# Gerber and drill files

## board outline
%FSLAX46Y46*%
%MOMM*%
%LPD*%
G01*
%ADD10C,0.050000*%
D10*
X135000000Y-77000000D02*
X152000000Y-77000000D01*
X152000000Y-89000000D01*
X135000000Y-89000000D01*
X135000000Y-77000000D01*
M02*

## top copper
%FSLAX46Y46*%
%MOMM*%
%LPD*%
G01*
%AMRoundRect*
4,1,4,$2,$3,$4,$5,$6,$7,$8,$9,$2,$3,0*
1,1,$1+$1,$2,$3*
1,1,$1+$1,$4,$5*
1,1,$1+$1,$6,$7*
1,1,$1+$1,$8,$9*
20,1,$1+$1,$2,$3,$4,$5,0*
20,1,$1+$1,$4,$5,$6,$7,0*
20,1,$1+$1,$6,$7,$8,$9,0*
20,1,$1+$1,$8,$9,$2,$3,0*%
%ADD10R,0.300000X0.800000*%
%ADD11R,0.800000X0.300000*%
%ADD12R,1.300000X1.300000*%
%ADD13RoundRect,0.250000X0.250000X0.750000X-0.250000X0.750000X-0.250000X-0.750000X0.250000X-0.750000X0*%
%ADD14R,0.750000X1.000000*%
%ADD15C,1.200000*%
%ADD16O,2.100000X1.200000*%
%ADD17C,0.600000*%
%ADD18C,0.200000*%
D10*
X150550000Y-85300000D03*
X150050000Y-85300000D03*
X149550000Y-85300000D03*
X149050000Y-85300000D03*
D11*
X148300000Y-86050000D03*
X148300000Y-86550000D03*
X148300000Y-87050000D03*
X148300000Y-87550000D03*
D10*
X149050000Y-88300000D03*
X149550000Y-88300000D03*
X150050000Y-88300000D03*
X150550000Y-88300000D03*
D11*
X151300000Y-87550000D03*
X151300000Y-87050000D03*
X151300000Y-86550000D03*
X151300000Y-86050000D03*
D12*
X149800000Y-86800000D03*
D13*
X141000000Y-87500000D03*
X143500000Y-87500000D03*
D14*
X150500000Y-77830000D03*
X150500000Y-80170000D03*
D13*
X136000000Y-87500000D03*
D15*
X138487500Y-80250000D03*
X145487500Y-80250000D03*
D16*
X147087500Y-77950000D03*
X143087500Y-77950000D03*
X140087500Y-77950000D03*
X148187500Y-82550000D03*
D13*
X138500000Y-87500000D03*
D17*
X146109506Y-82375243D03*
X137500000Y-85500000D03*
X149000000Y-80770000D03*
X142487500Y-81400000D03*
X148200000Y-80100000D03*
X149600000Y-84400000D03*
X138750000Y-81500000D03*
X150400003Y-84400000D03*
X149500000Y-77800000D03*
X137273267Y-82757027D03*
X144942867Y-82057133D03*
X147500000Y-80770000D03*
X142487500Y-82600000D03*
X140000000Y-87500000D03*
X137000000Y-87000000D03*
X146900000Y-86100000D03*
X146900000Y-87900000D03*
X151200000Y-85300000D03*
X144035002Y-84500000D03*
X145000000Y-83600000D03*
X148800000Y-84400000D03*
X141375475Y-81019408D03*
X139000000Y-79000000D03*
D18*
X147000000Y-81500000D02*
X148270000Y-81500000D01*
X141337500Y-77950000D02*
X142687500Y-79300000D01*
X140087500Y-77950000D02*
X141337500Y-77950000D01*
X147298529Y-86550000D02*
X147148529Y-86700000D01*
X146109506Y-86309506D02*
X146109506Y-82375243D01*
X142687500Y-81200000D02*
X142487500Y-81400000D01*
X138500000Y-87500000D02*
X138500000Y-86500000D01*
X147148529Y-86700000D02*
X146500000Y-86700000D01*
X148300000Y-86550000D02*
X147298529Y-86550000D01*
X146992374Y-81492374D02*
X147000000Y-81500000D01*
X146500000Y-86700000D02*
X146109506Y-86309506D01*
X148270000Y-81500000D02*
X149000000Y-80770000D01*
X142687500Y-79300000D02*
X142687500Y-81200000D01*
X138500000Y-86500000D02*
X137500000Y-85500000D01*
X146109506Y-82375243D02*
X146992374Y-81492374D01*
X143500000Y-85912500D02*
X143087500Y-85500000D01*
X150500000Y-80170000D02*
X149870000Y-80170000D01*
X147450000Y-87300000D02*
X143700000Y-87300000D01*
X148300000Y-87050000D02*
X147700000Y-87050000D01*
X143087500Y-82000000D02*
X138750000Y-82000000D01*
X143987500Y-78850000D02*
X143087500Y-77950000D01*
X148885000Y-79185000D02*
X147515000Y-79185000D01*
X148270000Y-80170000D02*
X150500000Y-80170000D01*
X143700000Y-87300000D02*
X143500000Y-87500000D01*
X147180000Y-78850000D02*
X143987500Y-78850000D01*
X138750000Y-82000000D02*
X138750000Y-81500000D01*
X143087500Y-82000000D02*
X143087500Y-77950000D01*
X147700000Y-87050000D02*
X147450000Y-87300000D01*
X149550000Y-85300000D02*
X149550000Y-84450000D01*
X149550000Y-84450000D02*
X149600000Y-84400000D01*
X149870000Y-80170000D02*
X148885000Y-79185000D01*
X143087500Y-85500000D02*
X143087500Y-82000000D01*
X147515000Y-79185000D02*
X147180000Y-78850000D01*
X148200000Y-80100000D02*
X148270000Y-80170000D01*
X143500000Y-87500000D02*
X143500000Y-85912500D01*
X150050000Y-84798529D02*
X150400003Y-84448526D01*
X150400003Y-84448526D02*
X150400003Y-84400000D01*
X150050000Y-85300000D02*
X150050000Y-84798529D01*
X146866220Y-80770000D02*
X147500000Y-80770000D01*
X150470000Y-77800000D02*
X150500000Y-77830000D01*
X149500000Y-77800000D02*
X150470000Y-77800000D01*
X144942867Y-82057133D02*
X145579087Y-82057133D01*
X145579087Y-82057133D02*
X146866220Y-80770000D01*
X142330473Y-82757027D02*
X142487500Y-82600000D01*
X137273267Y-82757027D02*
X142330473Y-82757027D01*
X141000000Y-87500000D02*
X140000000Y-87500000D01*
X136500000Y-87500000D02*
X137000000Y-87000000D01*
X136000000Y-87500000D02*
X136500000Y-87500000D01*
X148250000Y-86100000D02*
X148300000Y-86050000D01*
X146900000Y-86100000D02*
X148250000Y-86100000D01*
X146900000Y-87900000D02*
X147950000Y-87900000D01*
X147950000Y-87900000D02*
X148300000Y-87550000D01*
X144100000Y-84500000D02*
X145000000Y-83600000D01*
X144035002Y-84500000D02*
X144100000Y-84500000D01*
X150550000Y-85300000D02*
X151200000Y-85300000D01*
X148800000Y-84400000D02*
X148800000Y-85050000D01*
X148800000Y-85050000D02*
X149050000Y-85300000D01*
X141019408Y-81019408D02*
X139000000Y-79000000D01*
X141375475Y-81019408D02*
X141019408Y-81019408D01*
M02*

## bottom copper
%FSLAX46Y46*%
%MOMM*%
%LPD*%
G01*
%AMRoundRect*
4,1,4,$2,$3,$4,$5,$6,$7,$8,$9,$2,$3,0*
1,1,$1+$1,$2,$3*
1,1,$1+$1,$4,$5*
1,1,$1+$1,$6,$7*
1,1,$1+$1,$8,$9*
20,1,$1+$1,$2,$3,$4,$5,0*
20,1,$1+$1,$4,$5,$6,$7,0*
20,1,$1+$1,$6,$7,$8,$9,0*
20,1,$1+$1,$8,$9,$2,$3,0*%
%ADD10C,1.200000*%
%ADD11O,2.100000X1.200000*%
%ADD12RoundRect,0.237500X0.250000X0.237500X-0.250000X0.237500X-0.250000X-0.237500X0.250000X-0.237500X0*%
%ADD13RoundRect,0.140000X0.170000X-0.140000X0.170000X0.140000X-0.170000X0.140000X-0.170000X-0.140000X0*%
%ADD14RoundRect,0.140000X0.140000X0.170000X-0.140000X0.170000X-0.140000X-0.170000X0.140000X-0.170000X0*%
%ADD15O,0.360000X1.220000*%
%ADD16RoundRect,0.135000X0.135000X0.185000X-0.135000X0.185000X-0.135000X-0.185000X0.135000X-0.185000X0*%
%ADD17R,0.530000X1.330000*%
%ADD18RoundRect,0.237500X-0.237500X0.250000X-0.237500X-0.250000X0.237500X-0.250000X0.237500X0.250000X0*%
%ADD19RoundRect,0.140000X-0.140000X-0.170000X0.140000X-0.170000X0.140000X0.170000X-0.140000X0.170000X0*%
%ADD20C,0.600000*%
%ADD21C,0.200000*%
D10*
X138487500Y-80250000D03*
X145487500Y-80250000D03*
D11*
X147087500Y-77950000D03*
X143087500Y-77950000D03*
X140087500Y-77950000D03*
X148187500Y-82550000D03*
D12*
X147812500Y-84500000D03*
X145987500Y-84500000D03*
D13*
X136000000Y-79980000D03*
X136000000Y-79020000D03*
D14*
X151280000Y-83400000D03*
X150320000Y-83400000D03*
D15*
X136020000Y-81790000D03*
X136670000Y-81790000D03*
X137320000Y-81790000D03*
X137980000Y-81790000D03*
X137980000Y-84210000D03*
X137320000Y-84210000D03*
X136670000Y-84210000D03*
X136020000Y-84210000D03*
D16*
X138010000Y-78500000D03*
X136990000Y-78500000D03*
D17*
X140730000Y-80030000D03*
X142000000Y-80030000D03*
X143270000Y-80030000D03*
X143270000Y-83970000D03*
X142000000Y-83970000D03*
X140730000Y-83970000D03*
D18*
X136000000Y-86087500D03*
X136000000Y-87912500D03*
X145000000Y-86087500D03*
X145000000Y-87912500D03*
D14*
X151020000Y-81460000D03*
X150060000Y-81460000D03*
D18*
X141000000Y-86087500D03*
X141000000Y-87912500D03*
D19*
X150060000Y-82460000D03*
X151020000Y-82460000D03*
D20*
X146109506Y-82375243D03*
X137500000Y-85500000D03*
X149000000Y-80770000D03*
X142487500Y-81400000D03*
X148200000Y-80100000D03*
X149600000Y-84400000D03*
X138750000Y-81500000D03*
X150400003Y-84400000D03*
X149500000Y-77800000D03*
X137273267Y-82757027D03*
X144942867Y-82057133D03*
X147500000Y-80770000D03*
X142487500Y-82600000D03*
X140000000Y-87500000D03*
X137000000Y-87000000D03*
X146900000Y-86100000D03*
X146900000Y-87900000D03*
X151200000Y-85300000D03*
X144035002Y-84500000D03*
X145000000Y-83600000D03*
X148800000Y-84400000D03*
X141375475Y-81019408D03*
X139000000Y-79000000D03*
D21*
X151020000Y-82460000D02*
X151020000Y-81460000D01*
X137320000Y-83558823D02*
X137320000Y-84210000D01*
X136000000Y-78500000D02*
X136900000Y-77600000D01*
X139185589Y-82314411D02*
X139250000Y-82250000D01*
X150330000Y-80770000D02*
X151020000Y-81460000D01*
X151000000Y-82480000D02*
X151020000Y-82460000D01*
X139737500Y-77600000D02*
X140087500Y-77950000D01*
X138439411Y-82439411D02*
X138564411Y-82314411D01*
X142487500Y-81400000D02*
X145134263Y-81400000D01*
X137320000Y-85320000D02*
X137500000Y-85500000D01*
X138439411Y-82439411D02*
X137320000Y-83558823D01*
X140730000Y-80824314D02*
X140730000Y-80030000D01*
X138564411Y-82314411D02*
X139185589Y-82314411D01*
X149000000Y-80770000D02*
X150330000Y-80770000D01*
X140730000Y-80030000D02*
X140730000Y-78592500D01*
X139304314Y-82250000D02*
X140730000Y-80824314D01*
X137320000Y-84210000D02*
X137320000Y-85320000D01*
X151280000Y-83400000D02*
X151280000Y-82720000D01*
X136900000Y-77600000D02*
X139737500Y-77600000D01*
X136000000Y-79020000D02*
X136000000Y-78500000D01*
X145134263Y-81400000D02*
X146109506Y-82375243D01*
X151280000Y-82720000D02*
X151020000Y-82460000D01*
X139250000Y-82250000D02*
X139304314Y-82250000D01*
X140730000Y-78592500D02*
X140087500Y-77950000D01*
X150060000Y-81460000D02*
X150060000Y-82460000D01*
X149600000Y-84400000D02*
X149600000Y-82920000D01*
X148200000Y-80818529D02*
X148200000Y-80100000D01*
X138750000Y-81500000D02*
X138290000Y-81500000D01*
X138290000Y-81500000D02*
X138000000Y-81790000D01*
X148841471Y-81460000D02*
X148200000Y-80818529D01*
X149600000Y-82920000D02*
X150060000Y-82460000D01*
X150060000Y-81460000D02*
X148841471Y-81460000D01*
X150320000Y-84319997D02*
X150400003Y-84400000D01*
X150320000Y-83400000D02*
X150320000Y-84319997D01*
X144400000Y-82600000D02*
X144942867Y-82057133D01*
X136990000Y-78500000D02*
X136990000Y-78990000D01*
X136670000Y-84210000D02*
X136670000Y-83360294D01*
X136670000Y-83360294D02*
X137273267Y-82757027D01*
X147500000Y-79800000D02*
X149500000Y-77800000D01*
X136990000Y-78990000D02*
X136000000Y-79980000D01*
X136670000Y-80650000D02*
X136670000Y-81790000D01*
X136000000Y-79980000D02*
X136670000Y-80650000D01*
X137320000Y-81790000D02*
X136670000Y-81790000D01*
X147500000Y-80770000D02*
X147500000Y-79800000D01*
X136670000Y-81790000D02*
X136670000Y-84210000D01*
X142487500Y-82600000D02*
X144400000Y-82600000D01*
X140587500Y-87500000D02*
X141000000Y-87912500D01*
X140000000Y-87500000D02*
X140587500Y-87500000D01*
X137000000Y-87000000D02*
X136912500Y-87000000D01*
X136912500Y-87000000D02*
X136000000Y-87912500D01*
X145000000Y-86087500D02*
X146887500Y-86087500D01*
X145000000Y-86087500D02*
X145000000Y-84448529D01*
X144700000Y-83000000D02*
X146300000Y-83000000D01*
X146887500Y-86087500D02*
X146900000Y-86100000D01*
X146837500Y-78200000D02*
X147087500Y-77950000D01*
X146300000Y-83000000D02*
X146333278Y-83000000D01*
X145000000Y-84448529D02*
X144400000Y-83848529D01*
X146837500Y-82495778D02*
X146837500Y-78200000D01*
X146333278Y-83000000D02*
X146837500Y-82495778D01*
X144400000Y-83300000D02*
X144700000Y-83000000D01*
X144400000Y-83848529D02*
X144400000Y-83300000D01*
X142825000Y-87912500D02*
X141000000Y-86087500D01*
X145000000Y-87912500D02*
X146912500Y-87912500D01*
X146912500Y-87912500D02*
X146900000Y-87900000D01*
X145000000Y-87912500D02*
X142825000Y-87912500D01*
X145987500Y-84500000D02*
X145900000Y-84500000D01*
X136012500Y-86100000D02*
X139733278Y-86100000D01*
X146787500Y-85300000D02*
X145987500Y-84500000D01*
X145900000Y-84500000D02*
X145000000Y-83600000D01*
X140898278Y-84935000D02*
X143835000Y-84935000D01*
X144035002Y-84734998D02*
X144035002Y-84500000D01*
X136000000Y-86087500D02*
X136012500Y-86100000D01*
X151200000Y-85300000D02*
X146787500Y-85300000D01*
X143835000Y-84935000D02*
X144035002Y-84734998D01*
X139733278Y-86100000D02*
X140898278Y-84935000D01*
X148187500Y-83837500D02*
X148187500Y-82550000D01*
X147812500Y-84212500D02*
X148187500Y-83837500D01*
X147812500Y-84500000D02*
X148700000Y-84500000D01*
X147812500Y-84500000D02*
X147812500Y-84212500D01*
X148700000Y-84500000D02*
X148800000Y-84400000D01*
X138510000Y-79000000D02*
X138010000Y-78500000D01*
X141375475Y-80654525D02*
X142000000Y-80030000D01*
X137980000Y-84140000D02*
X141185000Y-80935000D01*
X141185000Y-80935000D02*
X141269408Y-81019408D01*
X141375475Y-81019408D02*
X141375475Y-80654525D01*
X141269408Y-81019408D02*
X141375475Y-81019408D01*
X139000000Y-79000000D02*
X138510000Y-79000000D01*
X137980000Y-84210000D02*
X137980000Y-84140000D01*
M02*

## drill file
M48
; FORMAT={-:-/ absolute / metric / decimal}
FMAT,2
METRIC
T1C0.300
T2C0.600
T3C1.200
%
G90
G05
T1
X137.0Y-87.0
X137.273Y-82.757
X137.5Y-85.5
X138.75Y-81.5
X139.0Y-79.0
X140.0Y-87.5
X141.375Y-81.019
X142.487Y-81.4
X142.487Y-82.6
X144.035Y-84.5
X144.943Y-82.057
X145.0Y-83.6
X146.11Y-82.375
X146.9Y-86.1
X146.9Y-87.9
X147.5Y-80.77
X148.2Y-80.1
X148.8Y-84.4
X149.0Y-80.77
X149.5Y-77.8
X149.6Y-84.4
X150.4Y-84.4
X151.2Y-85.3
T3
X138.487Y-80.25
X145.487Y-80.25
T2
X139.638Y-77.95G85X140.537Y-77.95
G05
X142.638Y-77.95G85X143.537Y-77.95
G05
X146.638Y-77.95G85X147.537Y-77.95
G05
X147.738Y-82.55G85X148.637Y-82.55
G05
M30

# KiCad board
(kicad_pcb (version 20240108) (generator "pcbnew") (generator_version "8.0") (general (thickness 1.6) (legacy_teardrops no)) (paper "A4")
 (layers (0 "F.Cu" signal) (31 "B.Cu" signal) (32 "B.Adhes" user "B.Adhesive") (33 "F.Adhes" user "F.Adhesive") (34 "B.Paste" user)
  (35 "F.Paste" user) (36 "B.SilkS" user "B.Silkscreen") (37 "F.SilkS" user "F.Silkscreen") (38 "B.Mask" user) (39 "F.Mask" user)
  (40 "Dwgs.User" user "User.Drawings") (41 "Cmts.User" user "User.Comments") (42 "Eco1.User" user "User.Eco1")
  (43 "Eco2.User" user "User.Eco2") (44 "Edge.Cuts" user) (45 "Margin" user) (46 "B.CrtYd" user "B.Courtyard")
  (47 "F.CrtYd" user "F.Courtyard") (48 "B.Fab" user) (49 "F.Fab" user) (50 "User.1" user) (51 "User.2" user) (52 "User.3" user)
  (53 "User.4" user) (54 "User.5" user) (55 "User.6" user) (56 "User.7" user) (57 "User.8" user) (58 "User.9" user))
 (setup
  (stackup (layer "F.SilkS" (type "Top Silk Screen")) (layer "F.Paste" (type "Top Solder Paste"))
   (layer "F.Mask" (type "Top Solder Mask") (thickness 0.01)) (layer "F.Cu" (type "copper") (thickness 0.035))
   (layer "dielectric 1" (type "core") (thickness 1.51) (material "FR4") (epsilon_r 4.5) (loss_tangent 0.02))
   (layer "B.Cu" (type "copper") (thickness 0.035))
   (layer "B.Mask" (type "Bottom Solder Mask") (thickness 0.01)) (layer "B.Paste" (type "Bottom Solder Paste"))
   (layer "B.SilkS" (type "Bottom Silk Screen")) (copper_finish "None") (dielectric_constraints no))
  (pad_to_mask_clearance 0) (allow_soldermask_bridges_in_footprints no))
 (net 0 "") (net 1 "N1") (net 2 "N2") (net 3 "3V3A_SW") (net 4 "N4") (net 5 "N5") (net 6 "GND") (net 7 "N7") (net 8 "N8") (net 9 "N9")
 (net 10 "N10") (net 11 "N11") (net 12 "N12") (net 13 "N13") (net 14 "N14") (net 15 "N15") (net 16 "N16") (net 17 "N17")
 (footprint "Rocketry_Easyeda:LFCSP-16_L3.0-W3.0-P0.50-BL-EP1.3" (layer "F.Cu") (at 149.8 86.8 180)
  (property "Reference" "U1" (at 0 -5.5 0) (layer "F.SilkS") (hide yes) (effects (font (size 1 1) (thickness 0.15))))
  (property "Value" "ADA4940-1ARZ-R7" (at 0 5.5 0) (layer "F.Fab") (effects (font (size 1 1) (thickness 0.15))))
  (pad "1" smd rect (at -0.75 1.5) (size 0.3 0.8) (layers "F.Cu" "F.Paste" "F.Mask") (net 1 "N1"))
  (pad "2" smd rect (at -0.25 1.5) (size 0.3 0.8) (layers "F.Cu" "F.Paste" "F.Mask") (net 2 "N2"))
  (pad "3" smd rect (at 0.25 1.5) (size 0.3 0.8) (layers "F.Cu" "F.Paste" "F.Mask") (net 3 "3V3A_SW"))
  (pad "4" smd rect (at 0.75 1.5) (size 0.3 0.8) (layers "F.Cu" "F.Paste" "F.Mask") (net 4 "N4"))
  (pad "5" smd rect (at 1.5 0.75 270) (size 0.3 0.8) (layers "F.Cu" "F.Paste" "F.Mask") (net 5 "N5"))
  (pad "6" smd rect (at 1.5 0.25 270) (size 0.3 0.8) (layers "F.Cu" "F.Paste" "F.Mask") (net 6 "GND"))
  (pad "7" smd rect (at 1.5 -0.25 270) (size 0.3 0.8) (layers "F.Cu" "F.Paste" "F.Mask") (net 3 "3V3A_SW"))
  (pad "8" smd rect (at 1.5 -0.75 270) (size 0.3 0.8) (layers "F.Cu" "F.Paste" "F.Mask") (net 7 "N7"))
  (pad "9" smd rect (at 0.75 -1.5) (size 0.3 0.8) (layers "F.Cu" "F.Paste" "F.Mask"))
  (pad "10" smd rect (at 0.25 -1.5) (size 0.3 0.8) (layers "F.Cu" "F.Paste" "F.Mask"))
  (pad "11" smd rect (at -0.25 -1.5) (size 0.3 0.8) (layers "F.Cu" "F.Paste" "F.Mask"))
  (pad "12" smd rect (at -0.75 -1.5) (size 0.3 0.8) (layers "F.Cu" "F.Paste" "F.Mask"))
  (pad "13" smd rect (at -1.5 -0.75 270) (size 0.3 0.8) (layers "F.Cu" "F.Paste" "F.Mask"))
  (pad "14" smd rect (at -1.5 -0.25 270) (size 0.3 0.8) (layers "F.Cu" "F.Paste" "F.Mask"))
  (pad "15" smd rect (at -1.5 0.25 270) (size 0.3 0.8) (layers "F.Cu" "F.Paste" "F.Mask"))
  (pad "16" smd rect (at -1.5 0.75 270) (size 0.3 0.8) (layers "F.Cu" "F.Paste" "F.Mask"))
  (pad "17" smd rect (at 0 0) (size 1.3 1.3) (layers "F.Cu" "F.Paste" "F.Mask")))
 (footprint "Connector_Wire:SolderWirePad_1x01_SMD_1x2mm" (layer "F.Cu") (at 141 87.5 180)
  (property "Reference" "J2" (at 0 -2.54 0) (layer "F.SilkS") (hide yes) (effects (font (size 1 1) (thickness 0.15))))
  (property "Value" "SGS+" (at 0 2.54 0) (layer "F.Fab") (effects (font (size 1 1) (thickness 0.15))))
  (pad "1" smd roundrect (at 0 0 180) (size 1 2) (layers "F.Cu" "F.Paste" "F.Mask") (roundrect_rratio 0.25) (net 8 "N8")))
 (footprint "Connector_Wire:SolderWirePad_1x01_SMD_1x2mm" (layer "F.Cu") (at 143.5 87.5 180)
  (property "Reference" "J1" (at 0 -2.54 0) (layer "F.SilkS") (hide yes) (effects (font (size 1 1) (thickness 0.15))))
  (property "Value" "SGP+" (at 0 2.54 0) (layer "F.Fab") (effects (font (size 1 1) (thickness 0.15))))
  (pad "1" smd roundrect (at 0 0 180) (size 1 2) (layers "F.Cu" "F.Paste" "F.Mask") (roundrect_rratio 0.25) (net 3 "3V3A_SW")))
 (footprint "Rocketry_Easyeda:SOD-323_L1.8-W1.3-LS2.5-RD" (layer "F.Cu") (at 150.5 79 -90)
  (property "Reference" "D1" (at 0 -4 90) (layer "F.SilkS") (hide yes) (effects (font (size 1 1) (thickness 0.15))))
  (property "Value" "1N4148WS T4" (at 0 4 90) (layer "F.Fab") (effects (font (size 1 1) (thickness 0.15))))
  (pad "1" smd rect (at -1.17 0 270) (size 1 0.75) (layers "F.Cu" "F.Paste" "F.Mask") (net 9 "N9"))
  (pad "2" smd rect (at 1.17 0 270) (size 1 0.75) (layers "F.Cu" "F.Paste" "F.Mask") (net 3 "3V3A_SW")))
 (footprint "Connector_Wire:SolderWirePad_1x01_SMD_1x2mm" (layer "F.Cu") (at 136 87.5 180)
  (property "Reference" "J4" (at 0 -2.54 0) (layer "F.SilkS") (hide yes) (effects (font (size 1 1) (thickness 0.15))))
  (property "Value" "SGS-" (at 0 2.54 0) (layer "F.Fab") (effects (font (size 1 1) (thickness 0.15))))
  (pad "1" smd roundrect (at 0 0 180) (size 1 2) (layers "F.Cu" "F.Paste" "F.Mask") (roundrect_rratio 0.25) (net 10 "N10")))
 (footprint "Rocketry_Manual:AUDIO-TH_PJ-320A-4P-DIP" (layer "F.Cu") (at 144.1375 80.25)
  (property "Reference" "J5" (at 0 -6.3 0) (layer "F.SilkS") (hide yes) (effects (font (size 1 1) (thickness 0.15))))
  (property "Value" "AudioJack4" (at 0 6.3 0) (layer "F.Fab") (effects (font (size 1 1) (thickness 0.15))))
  (pad "" thru_hole circle (at -5.65 0) (size 1.2 1.2) (drill 1.2) (layers "*.Cu" "*.Mask") (remove_unused_layers no))
  (pad "" thru_hole circle (at 1.35 0) (size 1.2 1.2) (drill 1.2) (layers "*.Cu" "*.Mask") (remove_unused_layers no))
  (pad "R1" thru_hole oval (at 2.95 -2.3 90) (size 1.2 2.1) (drill oval 0.599999 1.499997) (layers "*.Cu" "*.Mask")
   (remove_unused_layers no) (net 5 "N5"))
  (pad "R2" thru_hole oval (at -1.05 -2.3 90) (size 1.2 2.1) (drill oval 0.599999 1.499997) (layers "*.Cu" "*.Mask")
   (remove_unused_layers no) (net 3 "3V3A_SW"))
  (pad "S" thru_hole oval (at -4.05 -2.3 90) (size 1.2 2.1) (drill oval 0.599999 1.499997) (layers "*.Cu" "*.Mask")
   (remove_unused_layers no) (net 6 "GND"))
  (pad "T" thru_hole oval (at 4.05 2.3 90) (size 1.2 2.1) (drill oval 0.599999 1.499997) (layers "*.Cu" "*.Mask") (remove_unused_layers no)
   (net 4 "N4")))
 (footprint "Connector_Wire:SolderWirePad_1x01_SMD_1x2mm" (layer "F.Cu") (at 138.5 87.5 180)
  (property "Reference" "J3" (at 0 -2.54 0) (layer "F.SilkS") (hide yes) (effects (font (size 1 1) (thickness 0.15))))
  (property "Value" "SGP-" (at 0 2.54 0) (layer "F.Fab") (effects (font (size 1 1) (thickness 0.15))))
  (pad "1" smd roundrect (at 0 0 180) (size 1 2) (layers "F.Cu" "F.Paste" "F.Mask") (roundrect_rratio 0.25) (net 6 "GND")))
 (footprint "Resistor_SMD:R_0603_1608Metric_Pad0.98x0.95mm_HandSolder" (layer "B.Cu") (at 146.9 84.5 180)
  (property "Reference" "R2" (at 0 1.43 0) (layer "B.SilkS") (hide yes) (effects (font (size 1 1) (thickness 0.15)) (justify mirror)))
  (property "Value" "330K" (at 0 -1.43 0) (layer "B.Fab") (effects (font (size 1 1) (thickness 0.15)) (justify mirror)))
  (pad "1" smd roundrect (at -0.9125 0 180) (size 0.975 0.95) (layers "B.Cu" "B.Paste" "B.Mask") (roundrect_rratio 0.25) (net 4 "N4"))
  (pad "2" smd roundrect (at 0.9125 0 180) (size 0.975 0.95) (layers "B.Cu" "B.Paste" "B.Mask") (roundrect_rratio 0.25) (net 1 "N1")))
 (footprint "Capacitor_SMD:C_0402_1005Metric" (layer "B.Cu") (at 136 79.5 90)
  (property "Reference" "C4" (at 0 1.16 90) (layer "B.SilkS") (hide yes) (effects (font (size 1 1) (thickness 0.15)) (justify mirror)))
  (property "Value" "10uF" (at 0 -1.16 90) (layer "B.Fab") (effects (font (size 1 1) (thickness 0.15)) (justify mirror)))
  (pad "1" smd roundrect (at -0.48 0 90) (size 0.56 0.62) (layers "B.Cu" "B.Paste" "B.Mask") (roundrect_rratio 0.25) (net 9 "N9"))
  (pad "2" smd roundrect (at 0.48 0 90) (size 0.56 0.62) (layers "B.Cu" "B.Paste" "B.Mask") (roundrect_rratio 0.25) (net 6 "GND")))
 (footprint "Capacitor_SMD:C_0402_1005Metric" (layer "B.Cu") (at 150.8 83.4 180)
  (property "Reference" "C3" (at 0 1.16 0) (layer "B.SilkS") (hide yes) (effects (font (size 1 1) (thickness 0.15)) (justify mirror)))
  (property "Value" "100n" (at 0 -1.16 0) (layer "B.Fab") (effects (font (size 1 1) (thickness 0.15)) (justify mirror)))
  (pad "1" smd roundrect (at -0.48 0 180) (size 0.56 0.62) (layers "B.Cu" "B.Paste" "B.Mask") (roundrect_rratio 0.25) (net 6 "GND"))
  (pad "2" smd roundrect (at 0.48 0 180) (size 0.56 0.62) (layers "B.Cu" "B.Paste" "B.Mask") (roundrect_rratio 0.25) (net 2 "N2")))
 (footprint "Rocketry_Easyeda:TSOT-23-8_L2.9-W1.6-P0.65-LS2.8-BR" (layer "B.Cu") (at 137 83 90)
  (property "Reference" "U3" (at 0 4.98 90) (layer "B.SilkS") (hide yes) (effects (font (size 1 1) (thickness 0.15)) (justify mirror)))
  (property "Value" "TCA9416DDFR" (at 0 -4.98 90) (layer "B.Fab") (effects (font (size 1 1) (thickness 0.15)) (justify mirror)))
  (pad "1" smd oval (at 1.21 -0.98 90) (size 1.22 0.36) (layers "B.Cu" "B.Paste" "B.Mask") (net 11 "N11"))
  (pad "2" smd oval (at 1.21 -0.33 90) (size 1.22 0.36) (layers "B.Cu" "B.Paste" "B.Mask") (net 9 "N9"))
  (pad "3" smd oval (at 1.21 0.32 90) (size 1.22 0.36) (layers "B.Cu" "B.Paste" "B.Mask") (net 9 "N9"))
  (pad "4" smd oval (at 1.21 0.98 90) (size 1.22 0.36) (layers "B.Cu" "B.Paste" "B.Mask") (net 3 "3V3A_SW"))
  (pad "5" smd oval (at -1.21 0.98 90) (size 1.22 0.36) (layers "B.Cu" "B.Paste" "B.Mask") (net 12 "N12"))
  (pad "6" smd oval (at -1.21 0.32 90) (size 1.22 0.36) (layers "B.Cu" "B.Paste" "B.Mask") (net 6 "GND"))
  (pad "7" smd oval (at -1.21 -0.33 90) (size 1.22 0.36) (layers "B.Cu" "B.Paste" "B.Mask") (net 9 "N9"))
  (pad "8" smd oval (at -1.21 -0.98 90) (size 1.22 0.36) (layers "B.Cu" "B.Paste" "B.Mask") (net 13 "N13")))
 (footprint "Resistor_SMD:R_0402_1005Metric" (layer "B.Cu") (at 137.5 78.5 180)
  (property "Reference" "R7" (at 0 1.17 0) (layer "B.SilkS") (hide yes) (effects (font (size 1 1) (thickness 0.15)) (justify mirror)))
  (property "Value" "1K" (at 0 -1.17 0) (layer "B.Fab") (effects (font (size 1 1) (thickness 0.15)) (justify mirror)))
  (pad "1" smd roundrect (at -0.51 0 180) (size 0.54 0.64) (layers "B.Cu" "B.Paste" "B.Mask") (roundrect_rratio 0.25) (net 12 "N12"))
  (pad "2" smd roundrect (at 0.51 0 180) (size 0.54 0.64) (layers "B.Cu" "B.Paste" "B.Mask") (roundrect_rratio 0.25) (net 9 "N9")))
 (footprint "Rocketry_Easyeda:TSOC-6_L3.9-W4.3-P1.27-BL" (layer "B.Cu") (at 142 82)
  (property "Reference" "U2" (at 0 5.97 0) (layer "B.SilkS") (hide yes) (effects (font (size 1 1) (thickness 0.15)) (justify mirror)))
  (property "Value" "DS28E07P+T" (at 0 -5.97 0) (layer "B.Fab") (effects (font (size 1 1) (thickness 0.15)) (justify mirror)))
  (pad "1" smd rect (at -1.27 -1.97) (size 0.53 1.33) (layers "B.Cu" "B.Paste" "B.Mask") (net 6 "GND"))
  (pad "2" smd rect (at 0 -1.97) (size 0.53 1.33) (layers "B.Cu" "B.Paste" "B.Mask") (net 12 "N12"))
  (pad "3" smd rect (at 1.27 -1.97) (size 0.53 1.33) (layers "B.Cu" "B.Paste" "B.Mask") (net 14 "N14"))
  (pad "4" smd rect (at 1.27 1.97) (size 0.53 1.33) (layers "B.Cu" "B.Paste" "B.Mask") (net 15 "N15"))
  (pad "5" smd rect (at 0 1.97) (size 0.53 1.33) (layers "B.Cu" "B.Paste" "B.Mask") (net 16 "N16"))
  (pad "6" smd rect (at -1.27 1.97) (size 0.53 1.33) (layers "B.Cu" "B.Paste" "B.Mask") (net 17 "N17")))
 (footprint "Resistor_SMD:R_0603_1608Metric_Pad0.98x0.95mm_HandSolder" (layer "B.Cu") (at 136 87 -90)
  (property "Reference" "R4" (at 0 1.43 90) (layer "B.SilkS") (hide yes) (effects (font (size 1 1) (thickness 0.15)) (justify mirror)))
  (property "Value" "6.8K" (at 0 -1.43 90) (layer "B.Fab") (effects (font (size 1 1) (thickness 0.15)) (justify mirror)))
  (pad "1" smd roundrect (at -0.9125 0 270) (size 0.975 0.95) (layers "B.Cu" "B.Paste" "B.Mask") (roundrect_rratio 0.25) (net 1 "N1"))
  (pad "2" smd roundrect (at 0.9125 0 270) (size 0.975 0.95) (layers "B.Cu" "B.Paste" "B.Mask") (roundrect_rratio 0.25) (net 10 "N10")))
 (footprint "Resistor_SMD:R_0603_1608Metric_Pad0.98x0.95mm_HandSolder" (layer "B.Cu") (at 145 87 -90)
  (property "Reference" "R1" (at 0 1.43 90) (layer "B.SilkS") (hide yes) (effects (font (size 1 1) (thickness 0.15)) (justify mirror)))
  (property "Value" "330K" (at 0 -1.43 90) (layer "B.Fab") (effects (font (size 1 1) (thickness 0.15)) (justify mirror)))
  (pad "1" smd roundrect (at -0.9125 0 270) (size 0.975 0.95) (layers "B.Cu" "B.Paste" "B.Mask") (roundrect_rratio 0.25) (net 5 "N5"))
  (pad "2" smd roundrect (at 0.9125 0 270) (size 0.975 0.95) (layers "B.Cu" "B.Paste" "B.Mask") (roundrect_rratio 0.25) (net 7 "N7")))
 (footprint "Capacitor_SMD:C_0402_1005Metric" (layer "B.Cu") (at 150.54 81.46 180)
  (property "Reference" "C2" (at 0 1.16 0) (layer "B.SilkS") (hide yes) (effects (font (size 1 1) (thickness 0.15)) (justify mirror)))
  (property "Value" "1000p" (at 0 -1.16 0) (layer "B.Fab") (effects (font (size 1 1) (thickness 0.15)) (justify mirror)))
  (pad "1" smd roundrect (at -0.48 0 180) (size 0.56 0.62) (layers "B.Cu" "B.Paste" "B.Mask") (roundrect_rratio 0.25) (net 6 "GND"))
  (pad "2" smd roundrect (at 0.48 0 180) (size 0.56 0.62) (layers "B.Cu" "B.Paste" "B.Mask") (roundrect_rratio 0.25) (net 3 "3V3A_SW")))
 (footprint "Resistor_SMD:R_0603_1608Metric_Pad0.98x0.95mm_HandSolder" (layer "B.Cu") (at 141 87 -90)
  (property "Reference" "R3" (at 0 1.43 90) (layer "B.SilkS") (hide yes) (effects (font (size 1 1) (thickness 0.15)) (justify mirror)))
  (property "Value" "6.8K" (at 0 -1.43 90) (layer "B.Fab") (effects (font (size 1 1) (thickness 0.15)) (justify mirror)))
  (pad "1" smd roundrect (at -0.9125 0 270) (size 0.975 0.95) (layers "B.Cu" "B.Paste" "B.Mask") (roundrect_rratio 0.25) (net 7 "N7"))
  (pad "2" smd roundrect (at 0.9125 0 270) (size 0.975 0.95) (layers "B.Cu" "B.Paste" "B.Mask") (roundrect_rratio 0.25) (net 8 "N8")))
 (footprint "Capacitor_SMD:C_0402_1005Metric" (layer "B.Cu") (at 150.54 82.46)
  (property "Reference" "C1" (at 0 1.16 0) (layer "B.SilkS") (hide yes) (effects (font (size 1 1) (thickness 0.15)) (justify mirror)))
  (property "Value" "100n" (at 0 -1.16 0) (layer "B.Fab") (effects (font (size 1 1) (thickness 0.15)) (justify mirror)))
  (pad "1" smd roundrect (at -0.48 0) (size 0.56 0.62) (layers "B.Cu" "B.Paste" "B.Mask") (roundrect_rratio 0.25) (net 3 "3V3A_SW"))
  (pad "2" smd roundrect (at 0.48 0) (size 0.56 0.62) (layers "B.Cu" "B.Paste" "B.Mask") (roundrect_rratio 0.25) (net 6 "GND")))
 (gr_rect (start 135 77) (end 152 89) (stroke (width 0.05) (type default)) (fill none) (layer "Edge.Cuts"))
 (segment (start 147 81.5) (end 148.27 81.5) (width 0.2) (layer "F.Cu") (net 6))
 (segment (start 141.3375 77.95) (end 142.6875 79.3) (width 0.2) (layer "F.Cu") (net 6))
 (segment (start 140.0875 77.95) (end 141.3375 77.95) (width 0.2) (layer "F.Cu") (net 6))
 (segment (start 147.298529 86.55) (end 147.148529 86.7) (width 0.2) (layer "F.Cu") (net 6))
 (segment (start 146.109506 86.309506) (end 146.109506 82.375243) (width 0.2) (layer "F.Cu") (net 6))
 (segment (start 142.6875 81.2) (end 142.4875 81.4) (width 0.2) (layer "F.Cu") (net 6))
 (segment (start 138.5 87.5) (end 138.5 86.5) (width 0.2) (layer "F.Cu") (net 6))
 (segment (start 147.148529 86.7) (end 146.5 86.7) (width 0.2) (layer "F.Cu") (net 6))
 (segment (start 148.3 86.55) (end 147.298529 86.55) (width 0.2) (layer "F.Cu") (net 6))
 (segment (start 146.992374 81.492374) (end 147 81.5) (width 0.2) (layer "F.Cu") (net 6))
 (segment (start 146.5 86.7) (end 146.109506 86.309506) (width 0.2) (layer "F.Cu") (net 6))
 (segment (start 148.27 81.5) (end 149 80.77) (width 0.2) (layer "F.Cu") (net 6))
 (segment (start 142.6875 79.3) (end 142.6875 81.2) (width 0.2) (layer "F.Cu") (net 6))
 (segment (start 138.5 86.5) (end 137.5 85.5) (width 0.2) (layer "F.Cu") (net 6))
 (segment (start 146.109506 82.375243) (end 146.992374 81.492374) (width 0.2) (layer "F.Cu") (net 6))
 (via (at 146.109506 82.375243) (size 0.6) (drill 0.3) (layers "F.Cu" "B.Cu") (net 6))
 (via (at 137.5 85.5) (size 0.6) (drill 0.3) (layers "F.Cu" "B.Cu") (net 6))
 (via (at 149 80.77) (size 0.6) (drill 0.3) (layers "F.Cu" "B.Cu") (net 6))
 (via (at 142.4875 81.4) (size 0.6) (drill 0.3) (layers "F.Cu" "B.Cu") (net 6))
 (segment (start 151.02 82.46) (end 151.02 81.46) (width 0.2) (layer "B.Cu") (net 6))
 (segment (start 137.32 83.558823) (end 137.32 84.21) (width 0.2) (layer "B.Cu") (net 6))
 (segment (start 136 78.5) (end 136.9 77.6) (width 0.2) (layer "B.Cu") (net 6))
 (segment (start 139.185589 82.314411) (end 139.25 82.25) (width 0.2) (layer "B.Cu") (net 6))
 (segment (start 150.33 80.77) (end 151.02 81.46) (width 0.2) (layer "B.Cu") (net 6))
 (segment (start 151 82.48) (end 151.02 82.46) (width 0.2) (layer "B.Cu") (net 6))
 (segment (start 139.7375 77.6) (end 140.0875 77.95) (width 0.2) (layer "B.Cu") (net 6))
 (segment (start 138.439411 82.439411) (end 138.564411 82.314411) (width 0.2) (layer "B.Cu") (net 6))
 (segment (start 142.4875 81.4) (end 145.134263 81.4) (width 0.2) (layer "B.Cu") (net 6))
 (segment (start 137.32 85.32) (end 137.5 85.5) (width 0.2) (layer "B.Cu") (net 6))
 (segment (start 138.439411 82.439411) (end 137.32 83.558823) (width 0.2) (layer "B.Cu") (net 6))
 (segment (start 140.73 80.824314) (end 140.73 80.03) (width 0.2) (layer "B.Cu") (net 6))
 (segment (start 138.564411 82.314411) (end 139.185589 82.314411) (width 0.2) (layer "B.Cu") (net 6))
 (segment (start 149 80.77) (end 150.33 80.77) (width 0.2) (layer "B.Cu") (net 6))
 (segment (start 140.73 80.03) (end 140.73 78.5925) (width 0.2) (layer "B.Cu") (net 6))
 (segment (start 139.304314 82.25) (end 140.73 80.824314) (width 0.2) (layer "B.Cu") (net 6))
 (segment (start 137.32 84.21) (end 137.32 85.32) (width 0.2) (layer "B.Cu") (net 6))
 (segment (start 151.28 83.4) (end 151.28 82.72) (width 0.2) (layer "B.Cu") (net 6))
 (segment (start 136.9 77.6) (end 139.7375 77.6) (width 0.2) (layer "B.Cu") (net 6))
 (segment (start 136 79.02) (end 136 78.5) (width 0.2) (layer "B.Cu") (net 6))
 (segment (start 145.134263 81.4) (end 146.109506 82.375243) (width 0.2) (layer "B.Cu") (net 6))
 (segment (start 151.28 82.72) (end 151.02 82.46) (width 0.2) (layer "B.Cu") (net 6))
 (segment (start 139.25 82.25) (end 139.304314 82.25) (width 0.2) (layer "B.Cu") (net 6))
 (segment (start 140.73 78.5925) (end 140.0875 77.95) (width 0.2) (layer "B.Cu") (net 6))
 (segment (start 143.5 85.9125) (end 143.0875 85.5) (width 0.2) (layer "F.Cu") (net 3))
 (segment (start 150.5 80.17) (end 149.87 80.17) (width 0.2) (layer "F.Cu") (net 3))
 (segment (start 147.45 87.3) (end 143.7 87.3) (width 0.2) (layer "F.Cu") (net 3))
 (segment (start 148.3 87.05) (end 147.7 87.05) (width 0.2) (layer "F.Cu") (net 3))
 (segment (start 143.0875 82) (end 138.75 82) (width 0.2) (layer "F.Cu") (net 3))
 (segment (start 143.9875 78.85) (end 143.0875 77.95) (width 0.2) (layer "F.Cu") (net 3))
 (segment (start 148.885 79.185) (end 147.515 79.185) (width 0.2) (layer "F.Cu") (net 3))
 (segment (start 148.27 80.17) (end 150.5 80.17) (width 0.2) (layer "F.Cu") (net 3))
 (segment (start 143.7 87.3) (end 143.5 87.5) (width 0.2) (layer "F.Cu") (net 3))
 (segment (start 147.18 78.85) (end 143.9875 78.85) (width 0.2) (layer "F.Cu") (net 3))
 (segment (start 138.75 82) (end 138.75 81.5) (width 0.2) (layer "F.Cu") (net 3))
 (segment (start 143.0875 82) (end 143.0875 77.95) (width 0.2) (layer "F.Cu") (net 3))
 (segment (start 147.7 87.05) (end 147.45 87.3) (width 0.2) (layer "F.Cu") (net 3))
 (segment (start 149.55 85.3) (end 149.55 84.45) (width 0.2) (layer "F.Cu") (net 3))
 (segment (start 149.55 84.45) (end 149.6 84.4) (width 0.2) (layer "F.Cu") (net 3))
 (segment (start 149.87 80.17) (end 148.885 79.185) (width 0.2) (layer "F.Cu") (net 3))
 (segment (start 143.0875 85.5) (end 143.0875 82) (width 0.2) (layer "F.Cu") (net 3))
 (segment (start 147.515 79.185) (end 147.18 78.85) (width 0.2) (layer "F.Cu") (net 3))
 (segment (start 148.2 80.1) (end 148.27 80.17) (width 0.2) (layer "F.Cu") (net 3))
 (segment (start 143.5 87.5) (end 143.5 85.9125) (width 0.2) (layer "F.Cu") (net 3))
 (via (at 148.2 80.1) (size 0.6) (drill 0.3) (layers "F.Cu" "B.Cu") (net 3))
 (via (at 149.6 84.4) (size 0.6) (drill 0.3) (layers "F.Cu" "B.Cu") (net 3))
 (via (at 138.75 81.5) (size 0.6) (drill 0.3) (layers "F.Cu" "B.Cu") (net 3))
 (segment (start 150.06 81.46) (end 150.06 82.46) (width 0.2) (layer "B.Cu") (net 3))
 (segment (start 149.6 84.4) (end 149.6 82.92) (width 0.2) (layer "B.Cu") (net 3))
 (segment (start 148.2 80.818529) (end 148.2 80.1) (width 0.2) (layer "B.Cu") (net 3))
 (segment (start 138.75 81.5) (end 138.29 81.5) (width 0.2) (layer "B.Cu") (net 3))
 (segment (start 138.29 81.5) (end 138 81.79) (width 0.2) (layer "B.Cu") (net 3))
 (segment (start 148.841471 81.46) (end 148.2 80.818529) (width 0.2) (layer "B.Cu") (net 3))
 (segment (start 149.6 82.92) (end 150.06 82.46) (width 0.2) (layer "B.Cu") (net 3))
 (segment (start 150.06 81.46) (end 148.841471 81.46) (width 0.2) (layer "B.Cu") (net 3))
 (segment (start 150.05 84.798529) (end 150.400003 84.448526) (width 0.2) (layer "F.Cu") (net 2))
 (segment (start 150.400003 84.448526) (end 150.400003 84.4) (width 0.2) (layer "F.Cu") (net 2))
 (segment (start 150.05 85.3) (end 150.05 84.798529) (width 0.2) (layer "F.Cu") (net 2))
 (via (at 150.400003 84.4) (size 0.6) (drill 0.3) (layers "F.Cu" "B.Cu") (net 2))
 (segment (start 150.32 84.319997) (end 150.400003 84.4) (width 0.2) (layer "B.Cu") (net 2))
 (segment (start 150.32 83.4) (end 150.32 84.319997) (width 0.2) (layer "B.Cu") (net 2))
 (segment (start 146.86622 80.77) (end 147.5 80.77) (width 0.2) (layer "F.Cu") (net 9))
 (segment (start 150.47 77.8) (end 150.5 77.83) (width 0.2) (layer "F.Cu") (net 9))
 (segment (start 149.5 77.8) (end 150.47 77.8) (width 0.2) (layer "F.Cu") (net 9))
 (segment (start 144.942867 82.057133) (end 145.579087 82.057133) (width 0.2) (layer "F.Cu") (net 9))
 (segment (start 145.579087 82.057133) (end 146.86622 80.77) (width 0.2) (layer "F.Cu") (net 9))
 (segment (start 142.330473 82.757027) (end 142.4875 82.6) (width 0.2) (layer "F.Cu") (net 9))
 (segment (start 137.273267 82.757027) (end 142.330473 82.757027) (width 0.2) (layer "F.Cu") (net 9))
 (via (at 149.5 77.8) (size 0.6) (drill 0.3) (layers "F.Cu" "B.Cu") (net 9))
 (via (at 137.273267 82.757027) (size 0.6) (drill 0.3) (layers "F.Cu" "B.Cu") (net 9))
 (via (at 144.942867 82.057133) (size 0.6) (drill 0.3) (layers "F.Cu" "B.Cu") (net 9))
 (via (at 147.5 80.77) (size 0.6) (drill 0.3) (layers "F.Cu" "B.Cu") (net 9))
 (via (at 142.4875 82.6) (size 0.6) (drill 0.3) (layers "F.Cu" "B.Cu") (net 9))
 (segment (start 144.4 82.6) (end 144.942867 82.057133) (width 0.2) (layer "B.Cu") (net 9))
 (segment (start 136.99 78.5) (end 136.99 78.99) (width 0.2) (layer "B.Cu") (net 9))
 (segment (start 136.67 84.21) (end 136.67 83.360294) (width 0.2) (layer "B.Cu") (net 9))
 (segment (start 136.67 83.360294) (end 137.273267 82.757027) (width 0.2) (layer "B.Cu") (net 9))
 (segment (start 147.5 79.8) (end 149.5 77.8) (width 0.2) (layer "B.Cu") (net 9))
 (segment (start 136.99 78.99) (end 136 79.98) (width 0.2) (layer "B.Cu") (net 9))
 (segment (start 136.67 80.65) (end 136.67 81.79) (width 0.2) (layer "B.Cu") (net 9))
 (segment (start 136 79.98) (end 136.67 80.65) (width 0.2) (layer "B.Cu") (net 9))
 (segment (start 137.32 81.79) (end 136.67 81.79) (width 0.2) (layer "B.Cu") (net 9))
 (segment (start 147.5 80.77) (end 147.5 79.8) (width 0.2) (layer "B.Cu") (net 9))
 (segment (start 136.67 81.79) (end 136.67 84.21) (width 0.2) (layer "B.Cu") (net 9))
 (segment (start 142.4875 82.6) (end 144.4 82.6) (width 0.2) (layer "B.Cu") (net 9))
 (segment (start 141 87.5) (end 140 87.5) (width 0.2) (layer "F.Cu") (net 8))
 (via (at 140 87.5) (size 0.6) (drill 0.3) (layers "F.Cu" "B.Cu") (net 8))
 (segment (start 140.5875 87.5) (end 141 87.9125) (width 0.2) (layer "B.Cu") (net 8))
 (segment (start 140 87.5) (end 140.5875 87.5) (width 0.2) (layer "B.Cu") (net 8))
 (segment (start 136.5 87.5) (end 137 87) (width 0.2) (layer "F.Cu") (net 10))
 (segment (start 136 87.5) (end 136.5 87.5) (width 0.2) (layer "F.Cu") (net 10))
 (via (at 137 87) (size 0.6) (drill 0.3) (layers "F.Cu" "B.Cu") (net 10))
 (segment (start 137 87) (end 136.9125 87) (width 0.2) (layer "B.Cu") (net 10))
 (segment (start 136.9125 87) (end 136 87.9125) (width 0.2) (layer "B.Cu") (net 10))
 (segment (start 148.25 86.1) (end 148.3 86.05) (width 0.2) (layer "F.Cu") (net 5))
 (segment (start 146.9 86.1) (end 148.25 86.1) (width 0.2) (layer "F.Cu") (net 5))
 (via (at 146.9 86.1) (size 0.6) (drill 0.3) (layers "F.Cu" "B.Cu") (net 5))
 (segment (start 145 86.0875) (end 146.8875 86.0875) (width 0.2) (layer "B.Cu") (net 5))
 (segment (start 145 86.0875) (end 145 84.448529) (width 0.2) (layer "B.Cu") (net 5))
 (segment (start 144.7 83) (end 146.3 83) (width 0.2) (layer "B.Cu") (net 5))
 (segment (start 146.8875 86.0875) (end 146.9 86.1) (width 0.2) (layer "B.Cu") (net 5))
 (segment (start 146.8375 78.2) (end 147.0875 77.95) (width 0.2) (layer "B.Cu") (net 5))
 (segment (start 146.3 83) (end 146.333278 83) (width 0.2) (layer "B.Cu") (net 5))
 (segment (start 145 84.448529) (end 144.4 83.848529) (width 0.2) (layer "B.Cu") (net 5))
 (segment (start 146.8375 82.495778) (end 146.8375 78.2) (width 0.2) (layer "B.Cu") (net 5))
 (segment (start 146.333278 83) (end 146.8375 82.495778) (width 0.2) (layer "B.Cu") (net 5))
 (segment (start 144.4 83.3) (end 144.7 83) (width 0.2) (layer "B.Cu") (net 5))
 (segment (start 144.4 83.848529) (end 144.4 83.3) (width 0.2) (layer "B.Cu") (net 5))
 (segment (start 146.9 87.9) (end 147.95 87.9) (width 0.2) (layer "F.Cu") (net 7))
 (segment (start 147.95 87.9) (end 148.3 87.55) (width 0.2) (layer "F.Cu") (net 7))
 (via (at 146.9 87.9) (size 0.6) (drill 0.3) (layers "F.Cu" "B.Cu") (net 7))
 (segment (start 142.825 87.9125) (end 141 86.0875) (width 0.2) (layer "B.Cu") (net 7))
 (segment (start 145 87.9125) (end 146.9125 87.9125) (width 0.2) (layer "B.Cu") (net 7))
 (segment (start 146.9125 87.9125) (end 146.9 87.9) (width 0.2) (layer "B.Cu") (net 7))
 (segment (start 145 87.9125) (end 142.825 87.9125) (width 0.2) (layer "B.Cu") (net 7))
 (segment (start 144.1 84.5) (end 145 83.6) (width 0.2) (layer "F.Cu") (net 1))
 (segment (start 144.035002 84.5) (end 144.1 84.5) (width 0.2) (layer "F.Cu") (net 1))
 (segment (start 150.55 85.3) (end 151.2 85.3) (width 0.2) (layer "F.Cu") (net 1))
 (via (at 151.2 85.3) (size 0.6) (drill 0.3) (layers "F.Cu" "B.Cu") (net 1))
 (via (at 144.035002 84.5) (size 0.6) (drill 0.3) (layers "F.Cu" "B.Cu") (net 1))
 (via (at 145 83.6) (size 0.6) (drill 0.3) (layers "F.Cu" "B.Cu") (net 1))
 (segment (start 145.9875 84.5) (end 145.9 84.5) (width 0.2) (layer "B.Cu") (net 1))
 (segment (start 136.0125 86.1) (end 139.733278 86.1) (width 0.2) (layer "B.Cu") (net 1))
 (segment (start 146.7875 85.3) (end 145.9875 84.5) (width 0.2) (layer "B.Cu") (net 1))
 (segment (start 145.9 84.5) (end 145 83.6) (width 0.2) (layer "B.Cu") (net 1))
 (segment (start 140.898278 84.935) (end 143.835 84.935) (width 0.2) (layer "B.Cu") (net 1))
 (segment (start 144.035002 84.734998) (end 144.035002 84.5) (width 0.2) (layer "B.Cu") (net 1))
 (segment (start 136 86.0875) (end 136.0125 86.1) (width 0.2) (layer "B.Cu") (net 1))
 (segment (start 151.2 85.3) (end 146.7875 85.3) (width 0.2) (layer "B.Cu") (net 1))
 (segment (start 143.835 84.935) (end 144.035002 84.734998) (width 0.2) (layer "B.Cu") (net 1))
 (segment (start 139.733278 86.1) (end 140.898278 84.935) (width 0.2) (layer "B.Cu") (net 1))
 (segment (start 148.8 84.4) (end 148.8 85.05) (width 0.2) (layer "F.Cu") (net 4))
 (segment (start 148.8 85.05) (end 149.05 85.3) (width 0.2) (layer "F.Cu") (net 4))
 (via (at 148.8 84.4) (size 0.6) (drill 0.3) (layers "F.Cu" "B.Cu") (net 4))
 (segment (start 148.1875 83.8375) (end 148.1875 82.55) (width 0.2) (layer "B.Cu") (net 4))
 (segment (start 147.8125 84.2125) (end 148.1875 83.8375) (width 0.2) (layer "B.Cu") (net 4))
 (segment (start 147.8125 84.5) (end 148.7 84.5) (width 0.2) (layer "B.Cu") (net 4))
 (segment (start 147.8125 84.5) (end 147.8125 84.2125) (width 0.2) (layer "B.Cu") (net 4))
 (segment (start 148.7 84.5) (end 148.8 84.4) (width 0.2) (layer "B.Cu") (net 4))
 (segment (start 141.019408 81.019408) (end 139 79) (width 0.2) (layer "F.Cu") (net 12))
 (segment (start 141.375475 81.019408) (end 141.019408 81.019408) (width 0.2) (layer "F.Cu") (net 12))
 (via (at 141.375475 81.019408) (size 0.6) (drill 0.3) (layers "F.Cu" "B.Cu") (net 12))
 (via (at 139 79) (size 0.6) (drill 0.3) (layers "F.Cu" "B.Cu") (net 12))
 (segment (start 138.51 79) (end 138.01 78.5) (width 0.2) (layer "B.Cu") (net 12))
 (segment (start 141.375475 80.654525) (end 142 80.03) (width 0.2) (layer "B.Cu") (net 12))
 (segment (start 137.98 84.14) (end 141.185 80.935) (width 0.2) (layer "B.Cu") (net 12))
 (segment (start 141.185 80.935) (end 141.269408 81.019408) (width 0.2) (layer "B.Cu") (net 12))
 (segment (start 141.375475 81.019408) (end 141.375475 80.654525) (width 0.2) (layer "B.Cu") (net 12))
 (segment (start 141.269408 81.019408) (end 141.375475 81.019408) (width 0.2) (layer "B.Cu") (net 12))
 (segment (start 139 79) (end 138.51 79) (width 0.2) (layer "B.Cu") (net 12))
 (segment (start 137.98 84.21) (end 137.98 84.14) (width 0.2) (layer "B.Cu") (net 12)))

